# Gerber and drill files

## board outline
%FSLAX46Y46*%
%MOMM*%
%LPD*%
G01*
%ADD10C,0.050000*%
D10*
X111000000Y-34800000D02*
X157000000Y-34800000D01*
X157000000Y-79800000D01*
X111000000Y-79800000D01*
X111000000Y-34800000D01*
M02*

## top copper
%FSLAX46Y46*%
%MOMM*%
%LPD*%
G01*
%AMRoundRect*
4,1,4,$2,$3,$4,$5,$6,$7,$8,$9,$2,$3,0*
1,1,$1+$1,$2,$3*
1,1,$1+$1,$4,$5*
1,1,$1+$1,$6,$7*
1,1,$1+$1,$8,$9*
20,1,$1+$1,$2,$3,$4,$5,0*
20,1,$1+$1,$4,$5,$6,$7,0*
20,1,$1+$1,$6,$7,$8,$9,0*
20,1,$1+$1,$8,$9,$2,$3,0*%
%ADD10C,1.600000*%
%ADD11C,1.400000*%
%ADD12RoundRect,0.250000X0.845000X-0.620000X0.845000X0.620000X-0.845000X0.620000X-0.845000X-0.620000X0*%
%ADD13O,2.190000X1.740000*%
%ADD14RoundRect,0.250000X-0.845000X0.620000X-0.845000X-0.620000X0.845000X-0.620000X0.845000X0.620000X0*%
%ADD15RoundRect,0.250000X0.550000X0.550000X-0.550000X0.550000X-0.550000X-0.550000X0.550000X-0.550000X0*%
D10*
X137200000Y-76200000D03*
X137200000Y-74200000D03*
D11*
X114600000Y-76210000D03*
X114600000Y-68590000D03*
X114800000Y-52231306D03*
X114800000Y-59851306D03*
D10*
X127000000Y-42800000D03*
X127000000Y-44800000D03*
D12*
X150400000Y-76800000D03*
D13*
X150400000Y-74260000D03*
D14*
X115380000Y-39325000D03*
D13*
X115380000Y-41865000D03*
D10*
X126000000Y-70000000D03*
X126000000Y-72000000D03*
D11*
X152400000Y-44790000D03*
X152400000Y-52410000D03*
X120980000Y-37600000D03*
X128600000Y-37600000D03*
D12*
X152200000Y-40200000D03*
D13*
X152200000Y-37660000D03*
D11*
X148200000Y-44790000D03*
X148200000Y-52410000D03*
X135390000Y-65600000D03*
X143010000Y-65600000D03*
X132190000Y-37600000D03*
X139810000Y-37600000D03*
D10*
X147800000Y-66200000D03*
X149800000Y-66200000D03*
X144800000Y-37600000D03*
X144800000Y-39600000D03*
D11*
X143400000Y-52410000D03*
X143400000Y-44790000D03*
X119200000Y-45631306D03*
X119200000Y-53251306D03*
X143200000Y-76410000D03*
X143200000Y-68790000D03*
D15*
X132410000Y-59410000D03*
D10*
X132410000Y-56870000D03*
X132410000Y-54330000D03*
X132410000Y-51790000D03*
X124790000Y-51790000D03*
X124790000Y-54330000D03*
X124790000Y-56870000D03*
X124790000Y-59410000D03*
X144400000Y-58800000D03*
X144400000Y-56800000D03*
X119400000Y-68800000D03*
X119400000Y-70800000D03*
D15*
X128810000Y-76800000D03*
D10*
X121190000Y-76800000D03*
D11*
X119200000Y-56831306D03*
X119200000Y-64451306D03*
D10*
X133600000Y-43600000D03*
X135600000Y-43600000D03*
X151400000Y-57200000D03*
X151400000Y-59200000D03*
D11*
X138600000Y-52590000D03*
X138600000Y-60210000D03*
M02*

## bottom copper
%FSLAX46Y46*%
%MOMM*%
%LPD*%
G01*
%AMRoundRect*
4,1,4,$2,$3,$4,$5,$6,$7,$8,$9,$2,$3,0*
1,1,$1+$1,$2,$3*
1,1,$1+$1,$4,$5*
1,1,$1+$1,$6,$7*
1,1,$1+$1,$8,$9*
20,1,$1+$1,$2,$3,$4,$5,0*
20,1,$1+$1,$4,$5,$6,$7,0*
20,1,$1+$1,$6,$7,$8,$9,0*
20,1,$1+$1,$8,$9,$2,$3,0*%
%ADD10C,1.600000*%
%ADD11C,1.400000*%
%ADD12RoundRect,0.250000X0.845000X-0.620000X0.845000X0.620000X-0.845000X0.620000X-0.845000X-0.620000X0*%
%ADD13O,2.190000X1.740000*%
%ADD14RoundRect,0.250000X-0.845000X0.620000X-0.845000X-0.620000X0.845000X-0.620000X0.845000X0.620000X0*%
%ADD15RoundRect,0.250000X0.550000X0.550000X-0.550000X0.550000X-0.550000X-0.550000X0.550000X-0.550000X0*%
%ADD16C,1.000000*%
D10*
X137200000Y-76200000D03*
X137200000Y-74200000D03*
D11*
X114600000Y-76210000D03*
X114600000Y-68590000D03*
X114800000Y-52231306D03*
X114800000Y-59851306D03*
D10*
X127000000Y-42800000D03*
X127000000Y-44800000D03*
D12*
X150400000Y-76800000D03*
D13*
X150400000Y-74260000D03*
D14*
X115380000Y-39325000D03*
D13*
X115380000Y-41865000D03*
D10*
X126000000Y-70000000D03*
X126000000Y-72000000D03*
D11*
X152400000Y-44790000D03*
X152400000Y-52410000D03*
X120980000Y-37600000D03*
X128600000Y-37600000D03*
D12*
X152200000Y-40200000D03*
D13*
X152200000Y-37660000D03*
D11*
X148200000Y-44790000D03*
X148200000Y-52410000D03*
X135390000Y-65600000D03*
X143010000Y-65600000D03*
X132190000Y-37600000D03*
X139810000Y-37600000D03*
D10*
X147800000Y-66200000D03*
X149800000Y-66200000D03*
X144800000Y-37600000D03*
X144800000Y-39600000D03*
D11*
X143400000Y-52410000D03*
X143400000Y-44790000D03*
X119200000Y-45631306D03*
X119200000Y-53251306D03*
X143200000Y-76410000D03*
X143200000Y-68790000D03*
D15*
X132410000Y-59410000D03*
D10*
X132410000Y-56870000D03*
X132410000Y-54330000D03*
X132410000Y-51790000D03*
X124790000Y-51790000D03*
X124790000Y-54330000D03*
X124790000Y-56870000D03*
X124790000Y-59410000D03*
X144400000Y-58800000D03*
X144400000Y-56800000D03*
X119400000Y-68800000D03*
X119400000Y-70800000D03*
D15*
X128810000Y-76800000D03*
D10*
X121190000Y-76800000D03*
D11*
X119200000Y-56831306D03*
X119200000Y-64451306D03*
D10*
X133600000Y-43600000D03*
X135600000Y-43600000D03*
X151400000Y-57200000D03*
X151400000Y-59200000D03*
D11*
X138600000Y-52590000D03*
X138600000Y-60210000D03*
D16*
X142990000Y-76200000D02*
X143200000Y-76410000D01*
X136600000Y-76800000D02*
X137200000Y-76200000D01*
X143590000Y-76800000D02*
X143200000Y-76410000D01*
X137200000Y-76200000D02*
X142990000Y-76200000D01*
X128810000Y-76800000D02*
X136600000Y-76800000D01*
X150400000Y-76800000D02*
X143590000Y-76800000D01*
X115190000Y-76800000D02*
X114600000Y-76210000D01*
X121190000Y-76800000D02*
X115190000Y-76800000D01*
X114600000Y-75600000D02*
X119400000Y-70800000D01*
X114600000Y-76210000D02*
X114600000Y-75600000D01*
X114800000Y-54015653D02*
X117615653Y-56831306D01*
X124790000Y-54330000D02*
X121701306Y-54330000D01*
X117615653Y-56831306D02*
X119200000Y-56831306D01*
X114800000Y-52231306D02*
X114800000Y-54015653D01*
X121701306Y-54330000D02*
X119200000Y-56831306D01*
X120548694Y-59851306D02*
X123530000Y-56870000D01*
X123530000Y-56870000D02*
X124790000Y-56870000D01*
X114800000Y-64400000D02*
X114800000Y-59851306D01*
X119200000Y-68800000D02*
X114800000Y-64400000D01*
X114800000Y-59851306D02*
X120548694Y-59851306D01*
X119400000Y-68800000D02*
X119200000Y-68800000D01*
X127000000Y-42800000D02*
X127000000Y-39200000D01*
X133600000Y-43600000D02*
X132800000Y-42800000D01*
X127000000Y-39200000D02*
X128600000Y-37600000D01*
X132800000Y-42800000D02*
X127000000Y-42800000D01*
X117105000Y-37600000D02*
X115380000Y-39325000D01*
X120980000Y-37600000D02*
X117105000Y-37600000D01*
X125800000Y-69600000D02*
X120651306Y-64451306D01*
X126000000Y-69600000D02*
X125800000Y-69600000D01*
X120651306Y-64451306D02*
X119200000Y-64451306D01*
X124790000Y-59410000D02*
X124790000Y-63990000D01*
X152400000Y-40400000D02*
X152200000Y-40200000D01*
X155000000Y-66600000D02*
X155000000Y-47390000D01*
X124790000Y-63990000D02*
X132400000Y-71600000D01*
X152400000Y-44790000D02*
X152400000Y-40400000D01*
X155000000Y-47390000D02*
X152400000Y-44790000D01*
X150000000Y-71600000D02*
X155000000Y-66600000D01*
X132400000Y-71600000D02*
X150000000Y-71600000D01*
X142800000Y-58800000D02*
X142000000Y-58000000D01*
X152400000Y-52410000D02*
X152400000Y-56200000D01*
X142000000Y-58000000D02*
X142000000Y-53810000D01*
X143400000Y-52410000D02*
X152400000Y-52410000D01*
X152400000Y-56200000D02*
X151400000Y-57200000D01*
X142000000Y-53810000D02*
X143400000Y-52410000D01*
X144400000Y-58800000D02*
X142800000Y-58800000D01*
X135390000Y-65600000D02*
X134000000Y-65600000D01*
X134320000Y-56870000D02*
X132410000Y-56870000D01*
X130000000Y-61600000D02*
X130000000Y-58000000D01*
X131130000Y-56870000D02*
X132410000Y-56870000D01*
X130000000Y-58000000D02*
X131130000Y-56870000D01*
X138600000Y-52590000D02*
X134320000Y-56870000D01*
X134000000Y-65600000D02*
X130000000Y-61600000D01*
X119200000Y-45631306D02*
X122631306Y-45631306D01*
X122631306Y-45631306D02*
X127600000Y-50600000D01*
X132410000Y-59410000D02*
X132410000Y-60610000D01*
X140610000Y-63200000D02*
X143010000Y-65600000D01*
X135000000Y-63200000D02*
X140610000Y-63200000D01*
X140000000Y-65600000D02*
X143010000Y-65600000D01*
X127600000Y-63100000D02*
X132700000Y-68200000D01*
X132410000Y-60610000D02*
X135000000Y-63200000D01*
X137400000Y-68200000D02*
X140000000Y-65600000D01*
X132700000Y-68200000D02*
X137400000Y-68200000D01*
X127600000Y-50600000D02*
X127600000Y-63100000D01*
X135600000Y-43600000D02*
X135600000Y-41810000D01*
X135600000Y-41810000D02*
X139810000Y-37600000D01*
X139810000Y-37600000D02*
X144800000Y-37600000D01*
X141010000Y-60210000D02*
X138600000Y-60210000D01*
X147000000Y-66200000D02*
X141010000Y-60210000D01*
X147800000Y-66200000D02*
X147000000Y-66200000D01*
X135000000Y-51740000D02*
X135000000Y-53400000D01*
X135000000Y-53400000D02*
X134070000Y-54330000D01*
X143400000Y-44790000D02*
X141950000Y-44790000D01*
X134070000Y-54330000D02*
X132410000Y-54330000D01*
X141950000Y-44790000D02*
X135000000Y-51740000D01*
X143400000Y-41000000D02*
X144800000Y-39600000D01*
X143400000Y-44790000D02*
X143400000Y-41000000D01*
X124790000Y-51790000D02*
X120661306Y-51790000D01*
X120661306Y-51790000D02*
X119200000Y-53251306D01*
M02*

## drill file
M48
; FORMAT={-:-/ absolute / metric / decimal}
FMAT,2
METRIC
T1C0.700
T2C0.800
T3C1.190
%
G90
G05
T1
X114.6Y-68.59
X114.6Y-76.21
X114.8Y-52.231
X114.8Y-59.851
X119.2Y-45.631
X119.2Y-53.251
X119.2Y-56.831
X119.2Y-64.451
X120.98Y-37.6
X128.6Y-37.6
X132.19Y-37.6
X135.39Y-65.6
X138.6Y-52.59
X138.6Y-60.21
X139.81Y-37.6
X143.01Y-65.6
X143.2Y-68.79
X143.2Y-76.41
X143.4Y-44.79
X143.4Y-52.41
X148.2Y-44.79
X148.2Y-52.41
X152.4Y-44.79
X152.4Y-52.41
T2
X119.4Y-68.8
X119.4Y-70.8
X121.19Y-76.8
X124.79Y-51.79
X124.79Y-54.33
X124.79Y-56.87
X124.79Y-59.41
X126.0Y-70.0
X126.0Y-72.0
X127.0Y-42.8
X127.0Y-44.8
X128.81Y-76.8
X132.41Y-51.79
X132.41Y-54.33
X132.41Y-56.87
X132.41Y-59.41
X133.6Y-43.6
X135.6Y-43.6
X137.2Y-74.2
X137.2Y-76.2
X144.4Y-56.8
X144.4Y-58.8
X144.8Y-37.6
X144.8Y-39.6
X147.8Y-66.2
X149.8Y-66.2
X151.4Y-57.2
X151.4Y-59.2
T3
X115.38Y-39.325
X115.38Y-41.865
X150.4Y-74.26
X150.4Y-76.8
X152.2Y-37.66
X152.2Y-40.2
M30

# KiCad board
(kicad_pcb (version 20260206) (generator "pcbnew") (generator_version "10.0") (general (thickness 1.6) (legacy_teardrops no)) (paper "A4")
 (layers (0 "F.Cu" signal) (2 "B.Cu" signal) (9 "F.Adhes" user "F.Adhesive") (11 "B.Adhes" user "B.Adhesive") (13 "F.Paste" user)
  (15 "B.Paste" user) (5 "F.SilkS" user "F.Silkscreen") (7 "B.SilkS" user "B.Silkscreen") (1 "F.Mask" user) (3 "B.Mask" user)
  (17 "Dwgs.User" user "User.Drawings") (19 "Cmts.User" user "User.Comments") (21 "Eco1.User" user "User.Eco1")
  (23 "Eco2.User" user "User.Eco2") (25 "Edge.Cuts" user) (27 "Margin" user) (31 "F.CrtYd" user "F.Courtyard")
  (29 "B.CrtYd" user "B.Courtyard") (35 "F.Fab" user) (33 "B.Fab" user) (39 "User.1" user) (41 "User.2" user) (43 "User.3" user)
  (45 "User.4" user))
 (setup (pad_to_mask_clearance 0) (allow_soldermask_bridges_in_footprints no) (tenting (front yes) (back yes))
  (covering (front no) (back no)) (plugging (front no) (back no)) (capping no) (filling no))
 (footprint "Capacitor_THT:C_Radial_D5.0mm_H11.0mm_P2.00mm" (layer "F.Cu") (at 137.2 76.2 90)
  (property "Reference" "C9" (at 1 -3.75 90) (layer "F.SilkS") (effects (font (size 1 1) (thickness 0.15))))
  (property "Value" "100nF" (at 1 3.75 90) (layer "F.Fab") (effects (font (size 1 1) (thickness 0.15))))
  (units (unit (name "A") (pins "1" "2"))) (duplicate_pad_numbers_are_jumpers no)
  (pad "1" thru_hole circle (at 0 0 90) (size 1.6 1.6) (drill 0.8) (layers "*.Cu" "*.Mask") (remove_unused_layers no) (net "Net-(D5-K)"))
  (pad "2" thru_hole circle (at 2 0 90) (size 1.6 1.6) (drill 0.8) (layers "*.Cu" "*.Mask") (remove_unused_layers no) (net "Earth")))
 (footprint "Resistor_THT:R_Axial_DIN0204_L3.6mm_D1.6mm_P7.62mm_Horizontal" (layer "F.Cu") (at 114.6 76.21 90)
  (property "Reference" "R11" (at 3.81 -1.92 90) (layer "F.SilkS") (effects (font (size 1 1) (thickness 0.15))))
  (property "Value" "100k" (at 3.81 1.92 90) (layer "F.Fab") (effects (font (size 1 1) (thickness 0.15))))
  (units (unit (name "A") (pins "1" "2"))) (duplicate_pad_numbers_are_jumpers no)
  (pad "1" thru_hole circle (at 0 0 90) (size 1.4 1.4) (drill 0.7) (layers "*.Cu" "*.Mask") (remove_unused_layers no) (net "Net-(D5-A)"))
  (pad "2" thru_hole circle (at 7.62 0 90) (size 1.4 1.4) (drill 0.7) (layers "*.Cu" "*.Mask") (remove_unused_layers no) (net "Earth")))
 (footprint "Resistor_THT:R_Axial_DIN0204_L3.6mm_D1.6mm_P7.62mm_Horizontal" (layer "F.Cu") (at 114.8 52.231306 -90)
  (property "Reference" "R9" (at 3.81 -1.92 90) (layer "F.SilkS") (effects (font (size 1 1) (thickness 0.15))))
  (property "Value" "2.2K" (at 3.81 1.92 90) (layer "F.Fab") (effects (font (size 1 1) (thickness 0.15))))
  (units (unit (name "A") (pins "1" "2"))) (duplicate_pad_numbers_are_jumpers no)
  (pad "1" thru_hole circle (at 0 0 270) (size 1.4 1.4) (drill 0.7) (layers "*.Cu" "*.Mask") (remove_unused_layers no) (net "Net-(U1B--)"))
  (pad "2" thru_hole circle (at 7.62 0 270) (size 1.4 1.4) (drill 0.7) (layers "*.Cu" "*.Mask") (remove_unused_layers no)
   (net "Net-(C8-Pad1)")))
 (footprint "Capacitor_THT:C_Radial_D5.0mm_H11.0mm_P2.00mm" (layer "F.Cu") (at 127 42.8 -90)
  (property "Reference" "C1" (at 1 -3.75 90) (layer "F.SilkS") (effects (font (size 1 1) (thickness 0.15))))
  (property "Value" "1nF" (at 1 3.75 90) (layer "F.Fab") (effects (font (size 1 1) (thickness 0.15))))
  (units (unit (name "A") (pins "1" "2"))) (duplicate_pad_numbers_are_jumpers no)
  (pad "1" thru_hole circle (at 0 0 270) (size 1.6 1.6) (drill 0.8) (layers "*.Cu" "*.Mask") (remove_unused_layers no) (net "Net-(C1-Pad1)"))
  (pad "2" thru_hole circle (at 2 0 270) (size 1.6 1.6) (drill 0.8) (layers "*.Cu" "*.Mask") (remove_unused_layers no) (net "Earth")))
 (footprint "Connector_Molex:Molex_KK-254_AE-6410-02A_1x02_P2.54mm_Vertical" (layer "F.Cu") (at 150.4 76.8 90)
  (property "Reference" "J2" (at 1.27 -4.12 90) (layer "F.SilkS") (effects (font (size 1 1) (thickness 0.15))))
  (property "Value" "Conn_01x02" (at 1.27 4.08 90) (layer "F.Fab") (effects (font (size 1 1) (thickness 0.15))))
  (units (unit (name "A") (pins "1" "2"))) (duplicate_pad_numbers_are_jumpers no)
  (pad "1" thru_hole roundrect (at 0 0 90) (size 1.74 2.19) (drill 1.19) (layers "*.Cu" "*.Mask") (remove_unused_layers no)
   (roundrect_rratio 0.143678) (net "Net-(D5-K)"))
  (pad "2" thru_hole oval (at 2.54 0 90) (size 1.74 2.19) (drill 1.19) (layers "*.Cu" "*.Mask") (remove_unused_layers no) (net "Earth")))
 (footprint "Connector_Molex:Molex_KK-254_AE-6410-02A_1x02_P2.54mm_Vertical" (layer "F.Cu") (at 115.38 39.325 -90)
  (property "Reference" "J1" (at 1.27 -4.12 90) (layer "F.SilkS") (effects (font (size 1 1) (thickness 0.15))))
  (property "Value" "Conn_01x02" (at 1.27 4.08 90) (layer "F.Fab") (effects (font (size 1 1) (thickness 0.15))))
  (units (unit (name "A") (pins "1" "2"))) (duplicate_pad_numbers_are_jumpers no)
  (pad "1" thru_hole roundrect (at 0 0 270) (size 1.74 2.19) (drill 1.19) (layers "*.Cu" "*.Mask") (remove_unused_layers no)
   (roundrect_rratio 0.143678) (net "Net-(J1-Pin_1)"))
  (pad "2" thru_hole oval (at 2.54 0 270) (size 1.74 2.19) (drill 1.19) (layers "*.Cu" "*.Mask") (remove_unused_layers no) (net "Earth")))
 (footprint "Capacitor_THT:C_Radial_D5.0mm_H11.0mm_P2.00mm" (layer "F.Cu") (at 126 70 -90)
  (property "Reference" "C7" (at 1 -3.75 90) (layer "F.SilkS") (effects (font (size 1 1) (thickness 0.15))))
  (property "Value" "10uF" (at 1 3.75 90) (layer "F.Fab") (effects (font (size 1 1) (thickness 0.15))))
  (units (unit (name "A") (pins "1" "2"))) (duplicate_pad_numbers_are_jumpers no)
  (pad "1" thru_hole circle (at 0 0 270) (size 1.6 1.6) (drill 0.8) (layers "*.Cu" "*.Mask") (remove_unused_layers no) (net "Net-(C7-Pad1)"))
  (pad "2" thru_hole circle (at 2 0 270) (size 1.6 1.6) (drill 0.8) (layers "*.Cu" "*.Mask") (remove_unused_layers no) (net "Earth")))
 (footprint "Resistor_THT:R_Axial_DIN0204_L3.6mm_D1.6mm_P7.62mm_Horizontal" (layer "F.Cu") (at 152.4 44.79 -90)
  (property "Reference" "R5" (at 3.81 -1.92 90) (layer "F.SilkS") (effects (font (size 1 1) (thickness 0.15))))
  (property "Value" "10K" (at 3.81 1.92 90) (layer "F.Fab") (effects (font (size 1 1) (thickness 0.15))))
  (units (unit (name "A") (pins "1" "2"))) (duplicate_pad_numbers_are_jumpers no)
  (pad "1" thru_hole circle (at 0 0 270) (size 1.4 1.4) (drill 0.7) (layers "*.Cu" "*.Mask") (remove_unused_layers no) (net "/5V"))
  (pad "2" thru_hole circle (at 7.62 0 270) (size 1.4 1.4) (drill 0.7) (layers "*.Cu" "*.Mask") (remove_unused_layers no)
   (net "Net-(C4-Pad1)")))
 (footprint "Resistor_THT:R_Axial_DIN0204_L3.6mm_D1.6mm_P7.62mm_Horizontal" (layer "F.Cu") (at 120.98 37.6)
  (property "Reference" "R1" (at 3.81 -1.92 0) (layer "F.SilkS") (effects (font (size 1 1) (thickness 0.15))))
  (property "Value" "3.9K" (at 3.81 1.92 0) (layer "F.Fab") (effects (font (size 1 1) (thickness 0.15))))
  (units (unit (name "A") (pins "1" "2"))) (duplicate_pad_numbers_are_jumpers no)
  (pad "1" thru_hole circle (at 0 0) (size 1.4 1.4) (drill 0.7) (layers "*.Cu" "*.Mask") (remove_unused_layers no) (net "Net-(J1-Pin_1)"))
  (pad "2" thru_hole circle (at 7.62 0) (size 1.4 1.4) (drill 0.7) (layers "*.Cu" "*.Mask") (remove_unused_layers no) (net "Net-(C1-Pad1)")))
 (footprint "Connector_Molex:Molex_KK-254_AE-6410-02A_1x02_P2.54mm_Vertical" (layer "F.Cu") (at 152.2 40.2 90)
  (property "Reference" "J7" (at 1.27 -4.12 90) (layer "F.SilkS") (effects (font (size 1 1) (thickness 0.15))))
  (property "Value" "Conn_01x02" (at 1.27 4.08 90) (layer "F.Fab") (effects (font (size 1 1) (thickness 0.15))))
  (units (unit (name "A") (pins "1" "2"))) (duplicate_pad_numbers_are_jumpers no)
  (pad "1" thru_hole roundrect (at 0 0 90) (size 1.74 2.19) (drill 1.19) (layers "*.Cu" "*.Mask") (remove_unused_layers no)
   (roundrect_rratio 0.143678) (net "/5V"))
  (pad "2" thru_hole oval (at 2.54 0 90) (size 1.74 2.19) (drill 1.19) (layers "*.Cu" "*.Mask") (remove_unused_layers no) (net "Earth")))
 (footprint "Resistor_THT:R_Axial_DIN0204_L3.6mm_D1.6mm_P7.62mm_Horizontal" (layer "F.Cu") (at 148.2 44.79 -90)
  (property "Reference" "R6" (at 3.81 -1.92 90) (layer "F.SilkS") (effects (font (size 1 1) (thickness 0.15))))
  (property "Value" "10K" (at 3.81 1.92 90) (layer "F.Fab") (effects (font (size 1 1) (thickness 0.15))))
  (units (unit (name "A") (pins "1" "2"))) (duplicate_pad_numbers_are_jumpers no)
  (pad "1" thru_hole circle (at 0 0 270) (size 1.4 1.4) (drill 0.7) (layers "*.Cu" "*.Mask") (remove_unused_layers no) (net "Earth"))
  (pad "2" thru_hole circle (at 7.62 0 270) (size 1.4 1.4) (drill 0.7) (layers "*.Cu" "*.Mask") (remove_unused_layers no)
   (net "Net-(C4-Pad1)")))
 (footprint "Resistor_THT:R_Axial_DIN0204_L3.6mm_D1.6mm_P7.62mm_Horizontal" (layer "F.Cu") (at 135.39 65.6)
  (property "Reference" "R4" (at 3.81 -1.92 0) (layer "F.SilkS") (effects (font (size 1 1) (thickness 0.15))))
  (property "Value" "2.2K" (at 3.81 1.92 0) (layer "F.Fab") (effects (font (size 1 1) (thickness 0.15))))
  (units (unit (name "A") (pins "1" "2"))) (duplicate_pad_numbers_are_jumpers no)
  (pad "1" thru_hole circle (at 0 0) (size 1.4 1.4) (drill 0.7) (layers "*.Cu" "*.Mask") (remove_unused_layers no) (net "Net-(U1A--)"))
  (pad "2" thru_hole circle (at 7.62 0) (size 1.4 1.4) (drill 0.7) (layers "*.Cu" "*.Mask") (remove_unused_layers no) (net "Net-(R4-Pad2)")))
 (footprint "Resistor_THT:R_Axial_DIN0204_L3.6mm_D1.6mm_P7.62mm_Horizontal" (layer "F.Cu") (at 132.19 37.6)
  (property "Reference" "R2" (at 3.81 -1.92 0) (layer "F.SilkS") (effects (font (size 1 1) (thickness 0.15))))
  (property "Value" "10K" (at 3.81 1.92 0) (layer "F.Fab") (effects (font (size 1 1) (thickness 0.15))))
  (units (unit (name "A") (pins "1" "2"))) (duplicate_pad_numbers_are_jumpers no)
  (pad "1" thru_hole circle (at 0 0) (size 1.4 1.4) (drill 0.7) (layers "*.Cu" "*.Mask") (remove_unused_layers no) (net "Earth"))
  (pad "2" thru_hole circle (at 7.62 0) (size 1.4 1.4) (drill 0.7) (layers "*.Cu" "*.Mask") (remove_unused_layers no) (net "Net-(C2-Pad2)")))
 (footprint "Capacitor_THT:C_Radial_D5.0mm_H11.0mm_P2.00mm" (layer "F.Cu") (at 147.8 66.2)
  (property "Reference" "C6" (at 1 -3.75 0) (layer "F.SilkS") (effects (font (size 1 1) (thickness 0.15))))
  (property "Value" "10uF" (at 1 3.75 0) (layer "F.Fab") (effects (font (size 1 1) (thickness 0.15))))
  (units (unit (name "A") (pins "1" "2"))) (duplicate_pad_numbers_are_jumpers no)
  (pad "1" thru_hole circle (at 0 0) (size 1.6 1.6) (drill 0.8) (layers "*.Cu" "*.Mask") (remove_unused_layers no) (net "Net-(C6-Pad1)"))
  (pad "2" thru_hole circle (at 2 0) (size 1.6 1.6) (drill 0.8) (layers "*.Cu" "*.Mask") (remove_unused_layers no) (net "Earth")))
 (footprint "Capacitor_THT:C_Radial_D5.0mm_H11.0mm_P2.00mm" (layer "F.Cu") (at 144.8 37.6 -90)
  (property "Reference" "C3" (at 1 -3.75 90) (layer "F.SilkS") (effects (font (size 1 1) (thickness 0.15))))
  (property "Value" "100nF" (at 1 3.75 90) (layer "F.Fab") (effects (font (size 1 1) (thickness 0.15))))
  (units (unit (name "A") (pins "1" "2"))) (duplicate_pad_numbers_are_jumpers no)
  (pad "1" thru_hole circle (at 0 0 270) (size 1.6 1.6) (drill 0.8) (layers "*.Cu" "*.Mask") (remove_unused_layers no) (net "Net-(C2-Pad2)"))
  (pad "2" thru_hole circle (at 2 0 270) (size 1.6 1.6) (drill 0.8) (layers "*.Cu" "*.Mask") (remove_unused_layers no) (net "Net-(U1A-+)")))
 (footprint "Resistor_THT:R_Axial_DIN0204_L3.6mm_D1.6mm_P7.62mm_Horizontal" (layer "F.Cu") (at 143.4 52.41 90)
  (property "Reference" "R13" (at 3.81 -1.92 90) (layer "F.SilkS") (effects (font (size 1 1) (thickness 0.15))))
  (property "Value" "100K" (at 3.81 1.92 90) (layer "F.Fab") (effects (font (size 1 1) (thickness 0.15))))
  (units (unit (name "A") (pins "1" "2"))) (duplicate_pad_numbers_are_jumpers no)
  (pad "1" thru_hole circle (at 0 0 90) (size 1.4 1.4) (drill 0.7) (layers "*.Cu" "*.Mask") (remove_unused_layers no) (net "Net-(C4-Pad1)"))
  (pad "2" thru_hole circle (at 7.62 0 90) (size 1.4 1.4) (drill 0.7) (layers "*.Cu" "*.Mask") (remove_unused_layers no) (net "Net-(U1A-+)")))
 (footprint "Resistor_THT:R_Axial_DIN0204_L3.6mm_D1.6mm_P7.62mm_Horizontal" (layer "F.Cu") (at 119.2 45.631306 -90)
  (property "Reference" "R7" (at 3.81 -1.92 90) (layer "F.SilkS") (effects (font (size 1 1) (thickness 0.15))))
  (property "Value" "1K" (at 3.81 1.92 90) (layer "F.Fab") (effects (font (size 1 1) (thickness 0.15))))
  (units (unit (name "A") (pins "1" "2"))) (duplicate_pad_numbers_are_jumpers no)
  (pad "1" thru_hole circle (at 0 0 270) (size 1.4 1.4) (drill 0.7) (layers "*.Cu" "*.Mask") (remove_unused_layers no) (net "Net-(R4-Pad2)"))
  (pad "2" thru_hole circle (at 7.62 0 270) (size 1.4 1.4) (drill 0.7) (layers "*.Cu" "*.Mask") (remove_unused_layers no)
   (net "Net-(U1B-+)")))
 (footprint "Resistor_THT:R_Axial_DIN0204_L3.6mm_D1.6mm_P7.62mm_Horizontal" (layer "F.Cu") (at 143.2 76.41 90)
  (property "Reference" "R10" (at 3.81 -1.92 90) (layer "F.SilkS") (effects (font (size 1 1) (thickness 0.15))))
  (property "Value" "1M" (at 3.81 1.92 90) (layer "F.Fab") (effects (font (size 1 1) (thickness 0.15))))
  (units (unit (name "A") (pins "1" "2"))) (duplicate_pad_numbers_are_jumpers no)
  (pad "1" thru_hole circle (at 0 0 90) (size 1.4 1.4) (drill 0.7) (layers "*.Cu" "*.Mask") (remove_unused_layers no) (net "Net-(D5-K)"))
  (pad "2" thru_hole circle (at 7.62 0 90) (size 1.4 1.4) (drill 0.7) (layers "*.Cu" "*.Mask") (remove_unused_layers no) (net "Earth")))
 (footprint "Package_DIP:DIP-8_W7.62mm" (layer "F.Cu") (at 132.41 59.41 180)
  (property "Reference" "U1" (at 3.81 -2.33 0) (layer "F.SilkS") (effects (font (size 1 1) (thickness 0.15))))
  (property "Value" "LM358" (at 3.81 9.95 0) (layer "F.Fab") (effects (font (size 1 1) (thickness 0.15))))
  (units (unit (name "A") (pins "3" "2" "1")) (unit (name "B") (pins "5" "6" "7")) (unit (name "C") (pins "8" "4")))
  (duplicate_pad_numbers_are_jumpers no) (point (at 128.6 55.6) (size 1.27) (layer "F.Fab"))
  (pad "1" thru_hole roundrect (at 0 0 180) (size 1.6 1.6) (drill 0.8) (layers "*.Cu" "*.Mask") (remove_unused_layers no)
   (roundrect_rratio 0.15625) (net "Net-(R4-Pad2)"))
  (pad "2" thru_hole circle (at 0 2.54 180) (size 1.6 1.6) (drill 0.8) (layers "*.Cu" "*.Mask") (remove_unused_layers no)
   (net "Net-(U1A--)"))
  (pad "3" thru_hole circle (at 0 5.08 180) (size 1.6 1.6) (drill 0.8) (layers "*.Cu" "*.Mask") (remove_unused_layers no)
   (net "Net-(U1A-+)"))
  (pad "4" thru_hole circle (at 0 7.62 180) (size 1.6 1.6) (drill 0.8) (layers "*.Cu" "*.Mask") (remove_unused_layers no) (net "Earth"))
  (pad "5" thru_hole circle (at 7.62 7.62 180) (size 1.6 1.6) (drill 0.8) (layers "*.Cu" "*.Mask") (remove_unused_layers no)
   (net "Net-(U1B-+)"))
  (pad "6" thru_hole circle (at 7.62 5.08 180) (size 1.6 1.6) (drill 0.8) (layers "*.Cu" "*.Mask") (remove_unused_layers no)
   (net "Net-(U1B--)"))
  (pad "7" thru_hole circle (at 7.62 2.54 180) (size 1.6 1.6) (drill 0.8) (layers "*.Cu" "*.Mask") (remove_unused_layers no)
   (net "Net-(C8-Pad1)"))
  (pad "8" thru_hole circle (at 7.62 0 180) (size 1.6 1.6) (drill 0.8) (layers "*.Cu" "*.Mask") (remove_unused_layers no) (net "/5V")))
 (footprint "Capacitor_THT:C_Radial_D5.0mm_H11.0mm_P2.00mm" (layer "F.Cu") (at 144.4 58.8 90)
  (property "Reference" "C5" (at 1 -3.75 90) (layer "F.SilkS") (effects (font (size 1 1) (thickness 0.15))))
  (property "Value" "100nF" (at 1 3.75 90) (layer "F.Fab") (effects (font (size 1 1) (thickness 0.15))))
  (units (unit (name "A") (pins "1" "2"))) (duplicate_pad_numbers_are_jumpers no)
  (pad "1" thru_hole circle (at 0 0 90) (size 1.6 1.6) (drill 0.8) (layers "*.Cu" "*.Mask") (remove_unused_layers no) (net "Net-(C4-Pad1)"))
  (pad "2" thru_hole circle (at 2 0 90) (size 1.6 1.6) (drill 0.8) (layers "*.Cu" "*.Mask") (remove_unused_layers no) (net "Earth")))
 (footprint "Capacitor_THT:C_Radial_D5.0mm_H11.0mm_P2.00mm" (layer "F.Cu") (at 119.4 68.8 -90)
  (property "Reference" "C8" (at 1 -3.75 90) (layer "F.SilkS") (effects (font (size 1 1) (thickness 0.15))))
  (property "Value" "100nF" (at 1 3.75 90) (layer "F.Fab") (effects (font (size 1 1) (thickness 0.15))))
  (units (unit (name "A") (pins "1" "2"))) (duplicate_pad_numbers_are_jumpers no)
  (pad "1" thru_hole circle (at 0 0 270) (size 1.6 1.6) (drill 0.8) (layers "*.Cu" "*.Mask") (remove_unused_layers no) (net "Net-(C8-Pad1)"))
  (pad "2" thru_hole circle (at 2 0 270) (size 1.6 1.6) (drill 0.8) (layers "*.Cu" "*.Mask") (remove_unused_layers no) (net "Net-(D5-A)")))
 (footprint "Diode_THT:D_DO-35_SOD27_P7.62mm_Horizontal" (layer "F.Cu") (at 128.81 76.8 180)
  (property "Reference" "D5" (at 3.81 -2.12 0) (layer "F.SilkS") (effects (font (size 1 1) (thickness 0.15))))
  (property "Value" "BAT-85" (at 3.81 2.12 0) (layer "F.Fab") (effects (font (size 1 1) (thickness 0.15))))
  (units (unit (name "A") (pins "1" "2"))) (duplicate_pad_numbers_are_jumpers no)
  (pad "1" thru_hole roundrect (at 0 0 180) (size 1.6 1.6) (drill 0.8) (layers "*.Cu" "*.Mask") (remove_unused_layers no)
   (roundrect_rratio 0.15625) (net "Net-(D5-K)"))
  (pad "2" thru_hole circle (at 7.62 0 180) (size 1.6 1.6) (drill 0.8) (layers "*.Cu" "*.Mask") (remove_unused_layers no) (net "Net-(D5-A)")))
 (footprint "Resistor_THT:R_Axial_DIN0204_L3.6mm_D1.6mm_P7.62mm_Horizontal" (layer "F.Cu") (at 119.2 56.831306 -90)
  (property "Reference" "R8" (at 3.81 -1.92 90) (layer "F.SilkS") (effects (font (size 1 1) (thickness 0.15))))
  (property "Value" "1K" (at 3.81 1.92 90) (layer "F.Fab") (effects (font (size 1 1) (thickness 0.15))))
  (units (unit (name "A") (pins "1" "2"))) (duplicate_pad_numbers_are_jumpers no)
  (pad "1" thru_hole circle (at 0 0 270) (size 1.4 1.4) (drill 0.7) (layers "*.Cu" "*.Mask") (remove_unused_layers no) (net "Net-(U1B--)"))
  (pad "2" thru_hole circle (at 7.62 0 270) (size 1.4 1.4) (drill 0.7) (layers "*.Cu" "*.Mask") (remove_unused_layers no)
   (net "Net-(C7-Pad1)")))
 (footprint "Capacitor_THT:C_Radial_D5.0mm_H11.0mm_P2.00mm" (layer "F.Cu") (at 133.6 43.6)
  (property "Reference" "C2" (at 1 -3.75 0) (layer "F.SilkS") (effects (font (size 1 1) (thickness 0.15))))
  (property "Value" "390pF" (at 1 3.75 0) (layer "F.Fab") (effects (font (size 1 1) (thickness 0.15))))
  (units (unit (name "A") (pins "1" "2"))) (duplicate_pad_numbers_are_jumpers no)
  (pad "1" thru_hole circle (at 0 0) (size 1.6 1.6) (drill 0.8) (layers "*.Cu" "*.Mask") (remove_unused_layers no) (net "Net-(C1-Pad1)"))
  (pad "2" thru_hole circle (at 2 0) (size 1.6 1.6) (drill 0.8) (layers "*.Cu" "*.Mask") (remove_unused_layers no) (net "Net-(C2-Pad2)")))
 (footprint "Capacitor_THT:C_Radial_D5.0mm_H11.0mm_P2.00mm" (layer "F.Cu") (at 151.4 57.2 -90)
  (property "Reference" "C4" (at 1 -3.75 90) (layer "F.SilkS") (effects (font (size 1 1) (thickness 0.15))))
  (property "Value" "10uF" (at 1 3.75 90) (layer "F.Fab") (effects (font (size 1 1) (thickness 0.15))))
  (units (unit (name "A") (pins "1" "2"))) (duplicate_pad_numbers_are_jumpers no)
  (pad "1" thru_hole circle (at 0 0 270) (size 1.6 1.6) (drill 0.8) (layers "*.Cu" "*.Mask") (remove_unused_layers no) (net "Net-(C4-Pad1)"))
  (pad "2" thru_hole circle (at 2 0 270) (size 1.6 1.6) (drill 0.8) (layers "*.Cu" "*.Mask") (remove_unused_layers no) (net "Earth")))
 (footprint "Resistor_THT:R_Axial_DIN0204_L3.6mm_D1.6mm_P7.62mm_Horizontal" (layer "F.Cu") (at 138.6 52.59 -90)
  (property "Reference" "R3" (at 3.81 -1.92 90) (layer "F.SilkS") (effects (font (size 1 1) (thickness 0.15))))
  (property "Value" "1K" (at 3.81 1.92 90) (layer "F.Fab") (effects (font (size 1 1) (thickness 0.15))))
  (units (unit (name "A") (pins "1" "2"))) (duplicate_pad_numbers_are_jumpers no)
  (pad "1" thru_hole circle (at 0 0 270) (size 1.4 1.4) (drill 0.7) (layers "*.Cu" "*.Mask") (remove_unused_layers no) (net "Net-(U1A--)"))
  (pad "2" thru_hole circle (at 7.62 0 270) (size 1.4 1.4) (drill 0.7) (layers "*.Cu" "*.Mask") (remove_unused_layers no)
   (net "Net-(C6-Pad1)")))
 (gr_rect (start 111 34.8) (end 157 79.8) (stroke (width 0.05) (type solid)) (fill no) (layer "Edge.Cuts"))
 (segment (start 142.99 76.2) (end 143.2 76.41) (width 1) (layer "B.Cu") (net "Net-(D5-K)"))
 (segment (start 136.6 76.8) (end 137.2 76.2) (width 1) (layer "B.Cu") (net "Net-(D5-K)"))
 (segment (start 143.59 76.8) (end 143.2 76.41) (width 1) (layer "B.Cu") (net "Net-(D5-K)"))
 (segment (start 137.2 76.2) (end 142.99 76.2) (width 1) (layer "B.Cu") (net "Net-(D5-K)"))
 (segment (start 128.81 76.8) (end 136.6 76.8) (width 1) (layer "B.Cu") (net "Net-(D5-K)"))
 (segment (start 150.4 76.8) (end 143.59 76.8) (width 1) (layer "B.Cu") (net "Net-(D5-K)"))
 (segment (start 115.19 76.8) (end 114.6 76.21) (width 1) (layer "B.Cu") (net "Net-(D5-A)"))
 (segment (start 121.19 76.8) (end 115.19 76.8) (width 1) (layer "B.Cu") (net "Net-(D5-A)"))
 (segment (start 114.6 75.6) (end 119.4 70.8) (width 1) (layer "B.Cu") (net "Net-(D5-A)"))
 (segment (start 114.6 76.21) (end 114.6 75.6) (width 1) (layer "B.Cu") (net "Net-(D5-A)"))
 (segment (start 114.8 54.015653) (end 117.615653 56.831306) (width 1) (layer "B.Cu") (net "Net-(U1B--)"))
 (segment (start 124.79 54.33) (end 121.701306 54.33) (width 1) (layer "B.Cu") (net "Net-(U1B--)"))
 (segment (start 117.615653 56.831306) (end 119.2 56.831306) (width 1) (layer "B.Cu") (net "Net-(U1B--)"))
 (segment (start 114.8 52.231306) (end 114.8 54.015653) (width 1) (layer "B.Cu") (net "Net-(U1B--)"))
 (segment (start 121.701306 54.33) (end 119.2 56.831306) (width 1) (layer "B.Cu") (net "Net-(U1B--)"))
 (segment (start 120.548694 59.851306) (end 123.53 56.87) (width 1) (layer "B.Cu") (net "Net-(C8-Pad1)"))
 (segment (start 123.53 56.87) (end 124.79 56.87) (width 1) (layer "B.Cu") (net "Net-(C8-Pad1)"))
 (segment (start 114.8 64.4) (end 114.8 59.851306) (width 1) (layer "B.Cu") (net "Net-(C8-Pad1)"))
 (segment (start 119.2 68.8) (end 114.8 64.4) (width 1) (layer "B.Cu") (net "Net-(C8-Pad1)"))
 (segment (start 114.8 59.851306) (end 120.548694 59.851306) (width 1) (layer "B.Cu") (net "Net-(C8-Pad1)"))
 (segment (start 119.4 68.8) (end 119.2 68.8) (width 1) (layer "B.Cu") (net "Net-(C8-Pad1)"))
 (segment (start 127 42.8) (end 127 39.2) (width 1) (layer "B.Cu") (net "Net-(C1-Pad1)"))
 (segment (start 133.6 43.6) (end 132.8 42.8) (width 1) (layer "B.Cu") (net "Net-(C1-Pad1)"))
 (segment (start 127 39.2) (end 128.6 37.6) (width 1) (layer "B.Cu") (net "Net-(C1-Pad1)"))
 (segment (start 132.8 42.8) (end 127 42.8) (width 1) (layer "B.Cu") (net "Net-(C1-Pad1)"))
 (segment (start 117.105 37.6) (end 115.38 39.325) (width 1) (layer "B.Cu") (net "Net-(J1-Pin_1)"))
 (segment (start 120.98 37.6) (end 117.105 37.6) (width 1) (layer "B.Cu") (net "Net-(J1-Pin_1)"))
 (segment (start 125.8 69.6) (end 120.651306 64.451306) (width 1) (layer "B.Cu") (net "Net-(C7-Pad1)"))
 (segment (start 126 69.6) (end 125.8 69.6) (width 1) (layer "B.Cu") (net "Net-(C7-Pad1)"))
 (segment (start 120.651306 64.451306) (end 119.2 64.451306) (width 1) (layer "B.Cu") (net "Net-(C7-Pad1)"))
 (segment (start 124.79 59.41) (end 124.79 63.99) (width 1) (layer "B.Cu") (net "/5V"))
 (segment (start 152.4 40.4) (end 152.2 40.2) (width 1) (layer "B.Cu") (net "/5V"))
 (segment (start 155 66.6) (end 155 47.39) (width 1) (layer "B.Cu") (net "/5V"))
 (segment (start 124.79 63.99) (end 132.4 71.6) (width 1) (layer "B.Cu") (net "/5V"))
 (segment (start 152.4 44.79) (end 152.4 40.4) (width 1) (layer "B.Cu") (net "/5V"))
 (segment (start 155 47.39) (end 152.4 44.79) (width 1) (layer "B.Cu") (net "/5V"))
 (segment (start 150 71.6) (end 155 66.6) (width 1) (layer "B.Cu") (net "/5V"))
 (segment (start 132.4 71.6) (end 150 71.6) (width 1) (layer "B.Cu") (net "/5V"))
 (segment (start 142.8 58.8) (end 142 58) (width 1) (layer "B.Cu") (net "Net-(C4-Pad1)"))
 (segment (start 152.4 52.41) (end 152.4 56.2) (width 1) (layer "B.Cu") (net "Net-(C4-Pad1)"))
 (segment (start 142 58) (end 142 53.81) (width 1) (layer "B.Cu") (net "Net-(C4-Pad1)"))
 (segment (start 143.4 52.41) (end 152.4 52.41) (width 1) (layer "B.Cu") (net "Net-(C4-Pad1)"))
 (segment (start 152.4 56.2) (end 151.4 57.2) (width 1) (layer "B.Cu") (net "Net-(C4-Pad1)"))
 (segment (start 142 53.81) (end 143.4 52.41) (width 1) (layer "B.Cu") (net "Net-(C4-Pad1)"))
 (segment (start 144.4 58.8) (end 142.8 58.8) (width 1) (layer "B.Cu") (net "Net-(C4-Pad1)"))
 (segment (start 135.39 65.6) (end 134 65.6) (width 1) (layer "B.Cu") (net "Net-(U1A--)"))
 (segment (start 134.32 56.87) (end 132.41 56.87) (width 1) (layer "B.Cu") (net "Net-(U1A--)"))
 (segment (start 130 61.6) (end 130 58) (width 1) (layer "B.Cu") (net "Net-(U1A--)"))
 (segment (start 131.13 56.87) (end 132.41 56.87) (width 1) (layer "B.Cu") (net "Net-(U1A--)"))
 (segment (start 130 58) (end 131.13 56.87) (width 1) (layer "B.Cu") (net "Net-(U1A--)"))
 (segment (start 138.6 52.59) (end 134.32 56.87) (width 1) (layer "B.Cu") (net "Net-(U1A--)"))
 (segment (start 134 65.6) (end 130 61.6) (width 1) (layer "B.Cu") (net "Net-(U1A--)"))
 (segment (start 119.2 45.631306) (end 122.631306 45.631306) (width 1) (layer "B.Cu") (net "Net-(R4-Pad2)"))
 (segment (start 122.631306 45.631306) (end 127.6 50.6) (width 1) (layer "B.Cu") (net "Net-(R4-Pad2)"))
 (segment (start 132.41 59.41) (end 132.41 60.61) (width 1) (layer "B.Cu") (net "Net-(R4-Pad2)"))
 (segment (start 140.61 63.2) (end 143.01 65.6) (width 1) (layer "B.Cu") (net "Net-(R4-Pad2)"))
 (segment (start 135 63.2) (end 140.61 63.2) (width 1) (layer "B.Cu") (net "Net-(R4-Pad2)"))
 (segment (start 140 65.6) (end 143.01 65.6) (width 1) (layer "B.Cu") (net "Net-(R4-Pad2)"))
 (segment (start 127.6 63.1) (end 132.7 68.2) (width 1) (layer "B.Cu") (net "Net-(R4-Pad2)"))
 (segment (start 132.41 60.61) (end 135 63.2) (width 1) (layer "B.Cu") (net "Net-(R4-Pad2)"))
 (segment (start 137.4 68.2) (end 140 65.6) (width 1) (layer "B.Cu") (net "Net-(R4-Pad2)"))
 (segment (start 132.7 68.2) (end 137.4 68.2) (width 1) (layer "B.Cu") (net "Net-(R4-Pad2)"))
 (segment (start 127.6 50.6) (end 127.6 63.1) (width 1) (layer "B.Cu") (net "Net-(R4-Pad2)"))
 (segment (start 135.6 43.6) (end 135.6 41.81) (width 1) (layer "B.Cu") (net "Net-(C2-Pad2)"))
 (segment (start 135.6 41.81) (end 139.81 37.6) (width 1) (layer "B.Cu") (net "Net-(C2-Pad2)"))
 (segment (start 139.81 37.6) (end 144.8 37.6) (width 1) (layer "B.Cu") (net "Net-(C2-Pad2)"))
 (segment (start 141.01 60.21) (end 138.6 60.21) (width 1) (layer "B.Cu") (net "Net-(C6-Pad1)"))
 (segment (start 147 66.2) (end 141.01 60.21) (width 1) (layer "B.Cu") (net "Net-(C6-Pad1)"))
 (segment (start 147.8 66.2) (end 147 66.2) (width 1) (layer "B.Cu") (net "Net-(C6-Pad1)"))
 (segment (start 135 51.74) (end 135 53.4) (width 1) (layer "B.Cu") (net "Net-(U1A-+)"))
 (segment (start 135 53.4) (end 134.07 54.33) (width 1) (layer "B.Cu") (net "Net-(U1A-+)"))
 (segment (start 143.4 44.79) (end 141.95 44.79) (width 1) (layer "B.Cu") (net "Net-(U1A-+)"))
 (segment (start 134.07 54.33) (end 132.41 54.33) (width 1) (layer "B.Cu") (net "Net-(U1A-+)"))
 (segment (start 141.95 44.79) (end 135 51.74) (width 1) (layer "B.Cu") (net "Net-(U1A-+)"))
 (segment (start 143.4 41) (end 144.8 39.6) (width 1) (layer "B.Cu") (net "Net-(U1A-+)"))
 (segment (start 143.4 44.79) (end 143.4 41) (width 1) (layer "B.Cu") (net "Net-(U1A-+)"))
 (segment (start 124.79 51.79) (end 120.661306 51.79) (width 1) (layer "B.Cu") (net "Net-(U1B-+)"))
 (segment (start 120.661306 51.79) (end 119.2 53.251306) (width 1) (layer "B.Cu") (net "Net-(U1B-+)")))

